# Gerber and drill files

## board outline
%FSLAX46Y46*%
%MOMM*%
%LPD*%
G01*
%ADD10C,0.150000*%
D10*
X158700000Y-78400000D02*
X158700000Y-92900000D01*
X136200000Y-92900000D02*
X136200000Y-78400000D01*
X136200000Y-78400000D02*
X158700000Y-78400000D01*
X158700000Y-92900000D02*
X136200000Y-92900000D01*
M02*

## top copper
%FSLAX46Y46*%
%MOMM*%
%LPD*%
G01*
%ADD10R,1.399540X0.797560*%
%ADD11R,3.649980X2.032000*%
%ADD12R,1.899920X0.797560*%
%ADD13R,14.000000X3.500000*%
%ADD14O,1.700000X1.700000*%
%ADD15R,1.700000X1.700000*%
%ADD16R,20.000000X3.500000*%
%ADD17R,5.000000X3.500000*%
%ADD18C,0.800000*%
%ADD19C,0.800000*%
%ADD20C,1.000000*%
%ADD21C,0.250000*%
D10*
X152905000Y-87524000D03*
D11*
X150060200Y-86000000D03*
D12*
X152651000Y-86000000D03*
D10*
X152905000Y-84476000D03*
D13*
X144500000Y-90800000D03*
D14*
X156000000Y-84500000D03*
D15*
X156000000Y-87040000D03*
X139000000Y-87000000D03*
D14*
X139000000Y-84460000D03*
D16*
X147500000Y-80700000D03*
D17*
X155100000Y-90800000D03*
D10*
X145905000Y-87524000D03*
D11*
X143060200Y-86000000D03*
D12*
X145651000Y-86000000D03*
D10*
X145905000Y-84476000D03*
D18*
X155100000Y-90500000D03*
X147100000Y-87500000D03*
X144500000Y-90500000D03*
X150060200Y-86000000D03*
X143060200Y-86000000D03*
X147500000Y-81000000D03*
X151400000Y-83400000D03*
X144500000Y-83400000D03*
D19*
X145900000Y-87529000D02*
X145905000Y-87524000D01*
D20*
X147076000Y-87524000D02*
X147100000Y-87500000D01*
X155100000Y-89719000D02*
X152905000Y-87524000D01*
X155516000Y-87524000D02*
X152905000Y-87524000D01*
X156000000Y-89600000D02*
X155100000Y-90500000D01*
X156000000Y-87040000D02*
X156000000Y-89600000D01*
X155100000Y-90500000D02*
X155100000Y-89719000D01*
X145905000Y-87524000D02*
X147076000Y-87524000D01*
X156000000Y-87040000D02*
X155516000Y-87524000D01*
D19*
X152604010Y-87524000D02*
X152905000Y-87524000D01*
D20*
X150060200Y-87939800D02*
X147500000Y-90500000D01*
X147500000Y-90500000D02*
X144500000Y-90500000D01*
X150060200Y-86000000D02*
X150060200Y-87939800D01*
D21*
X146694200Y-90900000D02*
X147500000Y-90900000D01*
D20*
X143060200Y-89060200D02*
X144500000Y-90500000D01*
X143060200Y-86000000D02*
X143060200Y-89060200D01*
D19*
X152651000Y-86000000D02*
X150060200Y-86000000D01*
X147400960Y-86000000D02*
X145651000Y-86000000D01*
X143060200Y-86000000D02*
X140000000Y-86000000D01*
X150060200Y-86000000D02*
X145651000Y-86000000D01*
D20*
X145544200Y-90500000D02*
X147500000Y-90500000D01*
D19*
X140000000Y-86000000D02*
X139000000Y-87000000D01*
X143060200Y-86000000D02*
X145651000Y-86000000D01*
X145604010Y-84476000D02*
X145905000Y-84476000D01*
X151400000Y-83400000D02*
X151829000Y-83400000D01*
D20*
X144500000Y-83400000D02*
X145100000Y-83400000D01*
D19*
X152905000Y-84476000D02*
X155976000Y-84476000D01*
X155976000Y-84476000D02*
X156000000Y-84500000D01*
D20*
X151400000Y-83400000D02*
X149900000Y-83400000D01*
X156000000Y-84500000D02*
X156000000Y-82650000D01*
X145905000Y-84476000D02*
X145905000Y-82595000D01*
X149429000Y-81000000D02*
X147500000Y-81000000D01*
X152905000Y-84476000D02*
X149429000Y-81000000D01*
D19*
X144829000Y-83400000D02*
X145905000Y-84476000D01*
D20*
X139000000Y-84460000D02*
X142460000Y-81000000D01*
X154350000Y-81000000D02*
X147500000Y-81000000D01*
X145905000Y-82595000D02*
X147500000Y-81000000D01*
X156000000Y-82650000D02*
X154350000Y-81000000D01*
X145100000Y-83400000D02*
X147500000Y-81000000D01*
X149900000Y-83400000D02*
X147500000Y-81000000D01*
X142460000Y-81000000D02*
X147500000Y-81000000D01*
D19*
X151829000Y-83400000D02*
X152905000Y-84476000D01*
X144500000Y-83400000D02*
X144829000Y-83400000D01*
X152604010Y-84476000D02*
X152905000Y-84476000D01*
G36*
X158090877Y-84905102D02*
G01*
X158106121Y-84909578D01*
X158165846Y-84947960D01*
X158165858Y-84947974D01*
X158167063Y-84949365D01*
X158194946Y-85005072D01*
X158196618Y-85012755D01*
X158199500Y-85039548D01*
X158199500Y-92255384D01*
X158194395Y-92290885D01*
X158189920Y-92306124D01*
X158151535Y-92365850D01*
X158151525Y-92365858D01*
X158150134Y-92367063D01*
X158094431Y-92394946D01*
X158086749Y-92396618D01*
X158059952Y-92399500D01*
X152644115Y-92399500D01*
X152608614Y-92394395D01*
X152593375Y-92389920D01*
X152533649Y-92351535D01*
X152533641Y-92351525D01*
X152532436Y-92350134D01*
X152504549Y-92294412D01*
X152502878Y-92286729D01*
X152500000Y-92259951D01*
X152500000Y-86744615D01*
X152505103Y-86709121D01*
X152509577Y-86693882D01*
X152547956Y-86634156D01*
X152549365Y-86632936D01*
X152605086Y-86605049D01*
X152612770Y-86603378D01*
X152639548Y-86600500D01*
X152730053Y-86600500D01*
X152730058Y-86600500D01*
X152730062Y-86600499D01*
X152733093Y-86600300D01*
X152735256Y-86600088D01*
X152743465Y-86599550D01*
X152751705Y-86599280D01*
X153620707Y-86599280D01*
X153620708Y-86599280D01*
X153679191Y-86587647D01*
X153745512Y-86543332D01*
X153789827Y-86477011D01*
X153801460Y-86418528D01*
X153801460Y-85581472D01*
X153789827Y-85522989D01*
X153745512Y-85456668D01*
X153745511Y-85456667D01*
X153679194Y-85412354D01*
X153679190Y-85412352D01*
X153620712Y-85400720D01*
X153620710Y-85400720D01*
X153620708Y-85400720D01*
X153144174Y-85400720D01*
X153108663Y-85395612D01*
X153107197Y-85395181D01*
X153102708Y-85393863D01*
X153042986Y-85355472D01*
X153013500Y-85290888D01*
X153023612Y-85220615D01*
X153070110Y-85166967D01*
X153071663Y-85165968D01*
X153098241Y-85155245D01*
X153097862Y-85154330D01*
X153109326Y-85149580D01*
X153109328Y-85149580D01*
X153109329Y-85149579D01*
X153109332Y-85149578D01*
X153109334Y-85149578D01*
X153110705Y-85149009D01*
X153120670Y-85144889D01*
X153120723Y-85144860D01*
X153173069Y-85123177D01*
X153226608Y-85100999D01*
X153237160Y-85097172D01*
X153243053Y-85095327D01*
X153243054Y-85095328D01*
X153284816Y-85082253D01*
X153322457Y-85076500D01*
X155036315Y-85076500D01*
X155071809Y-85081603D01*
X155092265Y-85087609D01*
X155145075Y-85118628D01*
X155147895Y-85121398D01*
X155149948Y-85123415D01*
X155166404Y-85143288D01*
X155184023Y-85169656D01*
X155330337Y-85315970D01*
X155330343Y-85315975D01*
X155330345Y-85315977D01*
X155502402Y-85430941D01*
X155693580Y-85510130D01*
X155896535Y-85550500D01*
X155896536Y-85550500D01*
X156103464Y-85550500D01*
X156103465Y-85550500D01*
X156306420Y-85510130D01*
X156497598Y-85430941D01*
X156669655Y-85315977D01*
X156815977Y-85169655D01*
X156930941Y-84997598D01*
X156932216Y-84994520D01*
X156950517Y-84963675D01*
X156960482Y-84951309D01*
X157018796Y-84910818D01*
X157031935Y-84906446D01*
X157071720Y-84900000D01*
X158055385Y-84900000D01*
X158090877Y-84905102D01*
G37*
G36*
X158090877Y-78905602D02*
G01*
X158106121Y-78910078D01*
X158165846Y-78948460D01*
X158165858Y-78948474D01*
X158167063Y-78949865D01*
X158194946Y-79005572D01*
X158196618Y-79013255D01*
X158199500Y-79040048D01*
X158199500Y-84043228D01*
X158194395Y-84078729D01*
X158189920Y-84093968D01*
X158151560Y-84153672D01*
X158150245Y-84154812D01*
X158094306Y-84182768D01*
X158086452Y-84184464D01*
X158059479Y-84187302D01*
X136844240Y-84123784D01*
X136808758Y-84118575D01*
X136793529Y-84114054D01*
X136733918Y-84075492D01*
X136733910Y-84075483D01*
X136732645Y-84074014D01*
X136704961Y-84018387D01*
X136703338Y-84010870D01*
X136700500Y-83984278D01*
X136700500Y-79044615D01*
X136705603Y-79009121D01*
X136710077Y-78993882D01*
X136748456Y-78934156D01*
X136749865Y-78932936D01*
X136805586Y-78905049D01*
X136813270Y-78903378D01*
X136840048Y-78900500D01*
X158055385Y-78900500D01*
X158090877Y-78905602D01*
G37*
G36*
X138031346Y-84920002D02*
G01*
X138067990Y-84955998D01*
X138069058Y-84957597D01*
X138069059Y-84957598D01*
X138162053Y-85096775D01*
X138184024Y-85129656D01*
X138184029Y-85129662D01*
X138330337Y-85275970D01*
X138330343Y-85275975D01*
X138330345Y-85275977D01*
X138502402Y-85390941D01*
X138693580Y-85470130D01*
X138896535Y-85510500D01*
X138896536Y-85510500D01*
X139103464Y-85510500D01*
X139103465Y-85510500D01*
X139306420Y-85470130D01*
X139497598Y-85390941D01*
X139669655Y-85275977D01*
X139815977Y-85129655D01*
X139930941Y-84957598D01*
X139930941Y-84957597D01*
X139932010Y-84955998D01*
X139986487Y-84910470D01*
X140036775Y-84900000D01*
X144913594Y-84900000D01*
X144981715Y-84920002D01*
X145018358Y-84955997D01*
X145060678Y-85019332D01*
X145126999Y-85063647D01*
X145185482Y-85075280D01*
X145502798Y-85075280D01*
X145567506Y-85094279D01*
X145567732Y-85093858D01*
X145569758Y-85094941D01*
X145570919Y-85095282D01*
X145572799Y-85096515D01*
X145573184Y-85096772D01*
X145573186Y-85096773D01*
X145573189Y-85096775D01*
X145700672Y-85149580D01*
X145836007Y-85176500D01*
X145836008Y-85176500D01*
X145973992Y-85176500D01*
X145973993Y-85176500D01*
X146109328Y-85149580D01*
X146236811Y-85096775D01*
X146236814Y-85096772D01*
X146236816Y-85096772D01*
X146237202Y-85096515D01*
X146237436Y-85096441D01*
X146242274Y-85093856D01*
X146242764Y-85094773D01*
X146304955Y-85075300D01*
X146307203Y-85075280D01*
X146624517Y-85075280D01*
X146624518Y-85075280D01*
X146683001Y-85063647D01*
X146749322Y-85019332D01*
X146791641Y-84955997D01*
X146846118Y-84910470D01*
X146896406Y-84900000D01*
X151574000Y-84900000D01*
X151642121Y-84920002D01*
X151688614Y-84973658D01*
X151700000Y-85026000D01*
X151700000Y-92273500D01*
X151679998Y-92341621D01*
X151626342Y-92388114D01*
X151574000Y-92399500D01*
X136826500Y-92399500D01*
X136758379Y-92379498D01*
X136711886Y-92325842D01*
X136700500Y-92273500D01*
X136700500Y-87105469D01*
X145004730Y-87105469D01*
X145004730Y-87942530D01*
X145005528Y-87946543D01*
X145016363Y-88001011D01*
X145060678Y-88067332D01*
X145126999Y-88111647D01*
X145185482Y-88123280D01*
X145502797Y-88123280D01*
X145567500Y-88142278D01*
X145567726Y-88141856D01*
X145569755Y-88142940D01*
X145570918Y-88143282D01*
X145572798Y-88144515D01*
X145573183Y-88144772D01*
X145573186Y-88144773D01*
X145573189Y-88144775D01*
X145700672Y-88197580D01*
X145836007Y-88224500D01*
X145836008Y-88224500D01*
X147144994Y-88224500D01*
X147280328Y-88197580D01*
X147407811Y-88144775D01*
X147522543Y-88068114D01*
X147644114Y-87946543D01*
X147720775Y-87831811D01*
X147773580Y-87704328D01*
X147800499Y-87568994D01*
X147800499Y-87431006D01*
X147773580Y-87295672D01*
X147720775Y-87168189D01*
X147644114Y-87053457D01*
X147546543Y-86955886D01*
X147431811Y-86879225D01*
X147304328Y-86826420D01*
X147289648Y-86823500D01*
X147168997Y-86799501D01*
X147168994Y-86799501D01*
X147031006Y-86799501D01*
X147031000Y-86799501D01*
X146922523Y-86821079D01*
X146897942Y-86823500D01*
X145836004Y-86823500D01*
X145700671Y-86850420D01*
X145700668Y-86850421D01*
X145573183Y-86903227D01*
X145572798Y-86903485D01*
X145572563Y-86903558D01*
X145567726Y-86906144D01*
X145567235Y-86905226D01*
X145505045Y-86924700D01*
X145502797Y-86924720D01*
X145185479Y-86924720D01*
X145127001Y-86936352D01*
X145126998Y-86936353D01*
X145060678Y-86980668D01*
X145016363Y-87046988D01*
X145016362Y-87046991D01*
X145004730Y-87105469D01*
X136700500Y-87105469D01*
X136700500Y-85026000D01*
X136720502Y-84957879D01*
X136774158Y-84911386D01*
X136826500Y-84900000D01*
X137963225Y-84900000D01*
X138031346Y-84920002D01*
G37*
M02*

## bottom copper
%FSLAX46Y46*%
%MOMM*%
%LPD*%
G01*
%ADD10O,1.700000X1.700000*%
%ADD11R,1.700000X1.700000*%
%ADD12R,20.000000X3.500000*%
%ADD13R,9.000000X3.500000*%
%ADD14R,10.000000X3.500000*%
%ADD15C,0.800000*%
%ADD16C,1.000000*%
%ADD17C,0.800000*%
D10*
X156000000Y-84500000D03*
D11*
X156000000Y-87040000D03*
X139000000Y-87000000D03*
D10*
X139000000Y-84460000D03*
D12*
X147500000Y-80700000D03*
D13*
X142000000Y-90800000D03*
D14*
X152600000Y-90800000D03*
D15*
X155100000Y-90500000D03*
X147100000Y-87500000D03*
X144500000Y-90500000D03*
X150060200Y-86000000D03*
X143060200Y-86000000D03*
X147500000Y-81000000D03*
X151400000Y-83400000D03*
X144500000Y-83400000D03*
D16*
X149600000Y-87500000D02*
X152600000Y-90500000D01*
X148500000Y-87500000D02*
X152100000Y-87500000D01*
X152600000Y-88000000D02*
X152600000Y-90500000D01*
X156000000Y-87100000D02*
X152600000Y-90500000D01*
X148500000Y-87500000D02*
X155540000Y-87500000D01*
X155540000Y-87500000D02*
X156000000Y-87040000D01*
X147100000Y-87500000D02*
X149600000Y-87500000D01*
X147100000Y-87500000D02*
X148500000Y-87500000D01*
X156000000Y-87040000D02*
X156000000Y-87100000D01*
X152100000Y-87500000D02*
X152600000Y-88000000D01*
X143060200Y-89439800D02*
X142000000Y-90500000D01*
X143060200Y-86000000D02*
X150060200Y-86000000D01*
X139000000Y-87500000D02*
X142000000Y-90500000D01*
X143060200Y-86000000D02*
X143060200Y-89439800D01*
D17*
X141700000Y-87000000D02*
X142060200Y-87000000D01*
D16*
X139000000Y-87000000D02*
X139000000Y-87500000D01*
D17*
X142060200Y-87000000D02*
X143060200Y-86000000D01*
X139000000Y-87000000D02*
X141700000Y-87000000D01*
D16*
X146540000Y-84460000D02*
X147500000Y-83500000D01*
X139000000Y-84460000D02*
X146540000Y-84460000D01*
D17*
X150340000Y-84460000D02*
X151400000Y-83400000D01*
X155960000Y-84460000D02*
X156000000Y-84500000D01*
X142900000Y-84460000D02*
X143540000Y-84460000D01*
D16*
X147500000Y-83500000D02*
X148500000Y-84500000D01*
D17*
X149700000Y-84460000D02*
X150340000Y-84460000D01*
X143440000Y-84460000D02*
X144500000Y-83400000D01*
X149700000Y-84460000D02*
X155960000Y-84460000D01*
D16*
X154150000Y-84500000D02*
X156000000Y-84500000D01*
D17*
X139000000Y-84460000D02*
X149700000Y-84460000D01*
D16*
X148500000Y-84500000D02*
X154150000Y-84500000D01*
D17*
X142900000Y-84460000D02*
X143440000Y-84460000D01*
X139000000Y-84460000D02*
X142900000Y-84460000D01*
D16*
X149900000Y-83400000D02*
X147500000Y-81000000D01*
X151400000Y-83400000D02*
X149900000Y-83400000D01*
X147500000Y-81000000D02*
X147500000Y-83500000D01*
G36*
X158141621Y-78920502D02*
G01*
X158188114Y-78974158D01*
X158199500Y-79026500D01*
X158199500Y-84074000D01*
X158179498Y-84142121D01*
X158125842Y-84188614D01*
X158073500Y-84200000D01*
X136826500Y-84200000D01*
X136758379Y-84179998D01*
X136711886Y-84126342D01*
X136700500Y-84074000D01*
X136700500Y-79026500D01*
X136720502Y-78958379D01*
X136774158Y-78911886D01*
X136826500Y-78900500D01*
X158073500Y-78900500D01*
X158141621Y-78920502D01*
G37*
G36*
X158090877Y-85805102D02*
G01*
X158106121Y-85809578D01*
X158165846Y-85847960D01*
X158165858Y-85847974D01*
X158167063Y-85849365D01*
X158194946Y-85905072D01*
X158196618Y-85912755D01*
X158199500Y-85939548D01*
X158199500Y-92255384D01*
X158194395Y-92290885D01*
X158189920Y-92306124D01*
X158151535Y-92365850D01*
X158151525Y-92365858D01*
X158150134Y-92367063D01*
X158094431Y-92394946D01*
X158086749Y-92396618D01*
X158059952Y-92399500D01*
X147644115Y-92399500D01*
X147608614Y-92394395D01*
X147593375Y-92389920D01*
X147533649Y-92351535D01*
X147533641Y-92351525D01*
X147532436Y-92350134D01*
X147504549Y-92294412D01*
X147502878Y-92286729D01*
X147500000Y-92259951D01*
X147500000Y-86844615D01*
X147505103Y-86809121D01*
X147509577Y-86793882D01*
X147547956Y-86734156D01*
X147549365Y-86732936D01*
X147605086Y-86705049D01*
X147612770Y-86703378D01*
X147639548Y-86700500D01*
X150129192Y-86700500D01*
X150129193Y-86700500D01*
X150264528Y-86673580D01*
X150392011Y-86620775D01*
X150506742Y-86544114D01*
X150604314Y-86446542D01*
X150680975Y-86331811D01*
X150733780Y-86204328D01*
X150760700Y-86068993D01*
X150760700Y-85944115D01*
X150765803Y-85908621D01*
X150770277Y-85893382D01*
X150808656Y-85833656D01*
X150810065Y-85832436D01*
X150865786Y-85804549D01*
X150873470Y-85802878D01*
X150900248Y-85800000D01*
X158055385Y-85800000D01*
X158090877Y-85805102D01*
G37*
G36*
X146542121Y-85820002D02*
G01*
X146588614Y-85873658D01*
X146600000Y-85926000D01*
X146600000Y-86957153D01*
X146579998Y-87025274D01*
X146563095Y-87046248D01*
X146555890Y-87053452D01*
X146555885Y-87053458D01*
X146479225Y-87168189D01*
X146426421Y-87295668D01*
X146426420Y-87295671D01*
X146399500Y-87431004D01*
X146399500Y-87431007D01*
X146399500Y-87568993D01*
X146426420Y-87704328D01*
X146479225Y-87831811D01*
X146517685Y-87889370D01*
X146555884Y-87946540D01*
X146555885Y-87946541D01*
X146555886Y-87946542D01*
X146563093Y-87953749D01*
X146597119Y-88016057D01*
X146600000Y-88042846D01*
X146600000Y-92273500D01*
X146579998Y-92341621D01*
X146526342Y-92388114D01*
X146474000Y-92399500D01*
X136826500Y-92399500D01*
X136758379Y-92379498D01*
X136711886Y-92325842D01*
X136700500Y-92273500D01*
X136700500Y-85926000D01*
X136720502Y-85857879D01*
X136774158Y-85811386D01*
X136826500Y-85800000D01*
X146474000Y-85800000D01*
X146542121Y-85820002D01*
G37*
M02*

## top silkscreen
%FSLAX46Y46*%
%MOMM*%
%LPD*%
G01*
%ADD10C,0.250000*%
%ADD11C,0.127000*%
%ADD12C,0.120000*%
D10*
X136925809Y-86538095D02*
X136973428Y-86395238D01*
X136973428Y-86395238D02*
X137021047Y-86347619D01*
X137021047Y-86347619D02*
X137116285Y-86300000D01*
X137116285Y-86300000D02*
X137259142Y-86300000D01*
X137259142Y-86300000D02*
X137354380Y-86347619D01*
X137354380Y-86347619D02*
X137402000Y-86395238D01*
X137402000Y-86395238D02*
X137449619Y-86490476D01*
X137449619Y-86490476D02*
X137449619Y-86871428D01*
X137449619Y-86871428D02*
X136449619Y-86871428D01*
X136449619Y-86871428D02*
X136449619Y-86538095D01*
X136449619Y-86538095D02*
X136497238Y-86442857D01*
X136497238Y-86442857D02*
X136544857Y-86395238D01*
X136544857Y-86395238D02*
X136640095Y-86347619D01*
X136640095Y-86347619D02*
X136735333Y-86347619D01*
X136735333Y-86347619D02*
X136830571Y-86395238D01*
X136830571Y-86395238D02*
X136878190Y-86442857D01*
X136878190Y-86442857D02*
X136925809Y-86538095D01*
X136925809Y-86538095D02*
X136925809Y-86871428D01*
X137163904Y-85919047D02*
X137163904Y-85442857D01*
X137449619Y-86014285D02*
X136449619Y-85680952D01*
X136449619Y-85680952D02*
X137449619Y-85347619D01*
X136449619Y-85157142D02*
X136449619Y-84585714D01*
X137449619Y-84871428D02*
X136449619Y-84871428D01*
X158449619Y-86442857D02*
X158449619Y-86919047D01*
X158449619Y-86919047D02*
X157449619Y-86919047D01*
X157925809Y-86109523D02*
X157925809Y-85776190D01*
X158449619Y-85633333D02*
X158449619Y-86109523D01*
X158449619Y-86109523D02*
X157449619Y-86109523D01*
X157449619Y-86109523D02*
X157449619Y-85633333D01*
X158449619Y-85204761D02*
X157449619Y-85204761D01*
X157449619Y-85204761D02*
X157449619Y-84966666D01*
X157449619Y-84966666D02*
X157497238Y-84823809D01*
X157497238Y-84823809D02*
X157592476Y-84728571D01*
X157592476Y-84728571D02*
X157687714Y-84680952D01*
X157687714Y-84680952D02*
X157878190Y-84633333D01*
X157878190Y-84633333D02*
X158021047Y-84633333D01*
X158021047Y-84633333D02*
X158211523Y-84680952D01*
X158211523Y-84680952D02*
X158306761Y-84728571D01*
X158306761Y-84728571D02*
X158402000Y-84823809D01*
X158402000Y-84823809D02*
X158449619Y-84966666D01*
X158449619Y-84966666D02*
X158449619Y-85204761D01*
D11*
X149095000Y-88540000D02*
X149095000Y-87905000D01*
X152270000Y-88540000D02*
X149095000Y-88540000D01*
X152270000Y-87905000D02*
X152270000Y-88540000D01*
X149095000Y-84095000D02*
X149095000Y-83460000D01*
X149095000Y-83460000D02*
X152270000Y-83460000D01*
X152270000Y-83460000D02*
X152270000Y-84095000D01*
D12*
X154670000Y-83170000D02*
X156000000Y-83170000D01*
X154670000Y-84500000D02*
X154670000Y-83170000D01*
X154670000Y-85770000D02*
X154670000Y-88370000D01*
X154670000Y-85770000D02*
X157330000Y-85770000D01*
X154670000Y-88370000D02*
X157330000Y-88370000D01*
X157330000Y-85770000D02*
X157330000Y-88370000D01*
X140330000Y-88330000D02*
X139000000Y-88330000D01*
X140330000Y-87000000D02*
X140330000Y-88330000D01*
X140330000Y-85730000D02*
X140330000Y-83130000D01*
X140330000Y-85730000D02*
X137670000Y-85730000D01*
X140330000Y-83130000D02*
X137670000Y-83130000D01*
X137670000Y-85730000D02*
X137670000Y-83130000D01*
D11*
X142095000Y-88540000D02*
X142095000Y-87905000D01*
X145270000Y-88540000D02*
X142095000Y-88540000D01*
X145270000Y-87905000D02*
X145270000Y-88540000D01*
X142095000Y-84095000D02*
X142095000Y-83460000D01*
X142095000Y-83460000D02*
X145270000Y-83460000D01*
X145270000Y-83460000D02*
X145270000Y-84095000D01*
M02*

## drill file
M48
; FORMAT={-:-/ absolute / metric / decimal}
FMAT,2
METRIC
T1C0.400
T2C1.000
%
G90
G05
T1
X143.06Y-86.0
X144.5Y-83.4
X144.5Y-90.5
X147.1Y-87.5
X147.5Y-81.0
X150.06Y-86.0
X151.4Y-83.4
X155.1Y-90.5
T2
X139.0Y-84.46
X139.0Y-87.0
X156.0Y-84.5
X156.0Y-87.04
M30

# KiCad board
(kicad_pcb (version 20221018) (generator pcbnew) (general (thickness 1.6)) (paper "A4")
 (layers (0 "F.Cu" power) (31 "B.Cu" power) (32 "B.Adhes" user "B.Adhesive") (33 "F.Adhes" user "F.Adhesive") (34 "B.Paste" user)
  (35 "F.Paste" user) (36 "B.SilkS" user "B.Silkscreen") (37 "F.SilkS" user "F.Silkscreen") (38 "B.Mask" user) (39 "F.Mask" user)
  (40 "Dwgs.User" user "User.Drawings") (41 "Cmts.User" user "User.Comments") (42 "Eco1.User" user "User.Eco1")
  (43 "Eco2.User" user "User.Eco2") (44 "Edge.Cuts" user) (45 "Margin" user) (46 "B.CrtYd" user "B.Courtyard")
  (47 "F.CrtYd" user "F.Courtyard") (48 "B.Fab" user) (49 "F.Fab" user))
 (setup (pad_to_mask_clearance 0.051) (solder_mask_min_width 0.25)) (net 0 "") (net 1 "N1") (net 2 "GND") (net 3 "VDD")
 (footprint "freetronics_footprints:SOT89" (layer "F.Cu") (at 151 86 90)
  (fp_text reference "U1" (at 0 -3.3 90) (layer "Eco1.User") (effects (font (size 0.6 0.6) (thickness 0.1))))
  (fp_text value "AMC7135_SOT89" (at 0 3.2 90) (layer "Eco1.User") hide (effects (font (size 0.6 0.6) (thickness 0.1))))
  (fp_line (start -2.54 -1.905) (end -1.905 -1.905) (stroke (width 0.127) (type solid)) (layer "F.SilkS"))
  (fp_line (start -2.54 1.27) (end -2.54 -1.905) (stroke (width 0.127) (type solid)) (layer "F.SilkS"))
  (fp_line (start -1.905 1.27) (end -2.54 1.27) (stroke (width 0.127) (type solid)) (layer "F.SilkS"))
  (fp_line (start 1.905 -1.905) (end 2.54 -1.905) (stroke (width 0.127) (type solid)) (layer "F.SilkS"))
  (fp_line (start 2.54 -1.905) (end 2.54 1.27) (stroke (width 0.127) (type solid)) (layer "F.SilkS"))
  (fp_line (start 2.54 1.27) (end 1.905 1.27) (stroke (width 0.127) (type solid)) (layer "F.SilkS"))
  (pad "1" smd rect (at -1.524 1.905 90) (size 0.79756 1.39954) (layers "F.Cu" "F.Paste" "F.Mask") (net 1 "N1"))
  (pad "2" smd rect (at 0 -0.9398 90) (size 2.032 3.64998) (layers "F.Cu" "F.Paste" "F.Mask") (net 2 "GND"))
  (pad "2" smd rect (at 0 1.651 90) (size 0.79756 1.89992) (layers "F.Cu" "F.Paste" "F.Mask") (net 2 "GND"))
  (pad "3" smd rect (at 1.524 1.905 90) (size 0.79756 1.39954) (layers "F.Cu" "F.Paste" "F.Mask") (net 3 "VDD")))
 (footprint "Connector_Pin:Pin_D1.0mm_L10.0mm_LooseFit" (layer "F.Cu") (at 144.5 90.8)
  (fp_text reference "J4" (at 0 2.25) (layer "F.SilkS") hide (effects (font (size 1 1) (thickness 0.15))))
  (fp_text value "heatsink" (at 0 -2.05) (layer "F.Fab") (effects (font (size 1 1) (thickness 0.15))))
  (pad "1" smd rect (at 0 0) (size 14 3.5) (layers "F.Cu" "F.Paste" "F.Mask") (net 2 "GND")))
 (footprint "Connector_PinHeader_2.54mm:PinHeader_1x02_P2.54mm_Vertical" (layer "F.Cu") (at 156 84.5)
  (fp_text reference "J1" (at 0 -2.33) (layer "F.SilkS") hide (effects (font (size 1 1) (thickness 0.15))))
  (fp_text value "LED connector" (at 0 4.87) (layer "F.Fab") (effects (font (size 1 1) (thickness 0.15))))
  (fp_line (start -1.33 -1.33) (end 0 -1.33) (stroke (width 0.12) (type solid)) (layer "F.SilkS"))
  (fp_line (start -1.33 0) (end -1.33 -1.33) (stroke (width 0.12) (type solid)) (layer "F.SilkS"))
  (fp_line (start -1.33 1.27) (end -1.33 3.87) (stroke (width 0.12) (type solid)) (layer "F.SilkS"))
  (fp_line (start -1.33 1.27) (end 1.33 1.27) (stroke (width 0.12) (type solid)) (layer "F.SilkS"))
  (fp_line (start -1.33 3.87) (end 1.33 3.87) (stroke (width 0.12) (type solid)) (layer "F.SilkS"))
  (fp_line (start 1.33 1.27) (end 1.33 3.87) (stroke (width 0.12) (type solid)) (layer "F.SilkS"))
  (pad "1" thru_hole oval (at 0 0) (size 1.7 1.7) (drill 1) (layers "*.Cu" "*.Mask") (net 3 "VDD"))
  (pad "2" thru_hole rect (at 0 2.54) (size 1.7 1.7) (drill 1) (layers "*.Cu" "*.Mask") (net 1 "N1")))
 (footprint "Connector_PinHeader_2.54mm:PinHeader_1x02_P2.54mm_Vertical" (layer "F.Cu") (at 139 87 180)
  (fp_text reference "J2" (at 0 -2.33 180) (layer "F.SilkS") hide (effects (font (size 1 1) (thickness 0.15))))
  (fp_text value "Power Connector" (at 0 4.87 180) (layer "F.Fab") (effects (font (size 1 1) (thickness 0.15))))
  (fp_line (start -1.33 -1.33) (end 0 -1.33) (stroke (width 0.12) (type solid)) (layer "F.SilkS"))
  (fp_line (start -1.33 0) (end -1.33 -1.33) (stroke (width 0.12) (type solid)) (layer "F.SilkS"))
  (fp_line (start -1.33 1.27) (end -1.33 3.87) (stroke (width 0.12) (type solid)) (layer "F.SilkS"))
  (fp_line (start -1.33 1.27) (end 1.33 1.27) (stroke (width 0.12) (type solid)) (layer "F.SilkS"))
  (fp_line (start -1.33 3.87) (end 1.33 3.87) (stroke (width 0.12) (type solid)) (layer "F.SilkS"))
  (fp_line (start 1.33 1.27) (end 1.33 3.87) (stroke (width 0.12) (type solid)) (layer "F.SilkS"))
  (pad "1" thru_hole rect (at 0 0 180) (size 1.7 1.7) (drill 1) (layers "*.Cu" "*.Mask") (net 2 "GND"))
  (pad "2" thru_hole oval (at 0 2.54 180) (size 1.7 1.7) (drill 1) (layers "*.Cu" "*.Mask") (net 3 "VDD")))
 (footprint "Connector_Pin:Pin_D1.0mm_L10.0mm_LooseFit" (layer "F.Cu") (at 147.5 80.7)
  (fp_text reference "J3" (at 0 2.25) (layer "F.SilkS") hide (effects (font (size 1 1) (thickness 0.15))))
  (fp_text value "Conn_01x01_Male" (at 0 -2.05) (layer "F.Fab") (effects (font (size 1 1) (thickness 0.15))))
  (pad "1" smd rect (at 0 0) (size 20 3.5) (layers "F.Cu" "F.Paste" "F.Mask") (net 3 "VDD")))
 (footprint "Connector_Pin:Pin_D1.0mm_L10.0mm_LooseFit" (layer "F.Cu") (at 155.1 90.8)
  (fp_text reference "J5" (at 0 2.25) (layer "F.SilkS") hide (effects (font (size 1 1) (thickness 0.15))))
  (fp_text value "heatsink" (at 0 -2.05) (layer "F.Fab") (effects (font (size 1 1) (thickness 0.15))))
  (pad "1" smd rect (at 0 0) (size 5 3.5) (layers "F.Cu" "F.Paste" "F.Mask") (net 1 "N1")))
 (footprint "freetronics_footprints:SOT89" (layer "F.Cu") (at 144 86 90)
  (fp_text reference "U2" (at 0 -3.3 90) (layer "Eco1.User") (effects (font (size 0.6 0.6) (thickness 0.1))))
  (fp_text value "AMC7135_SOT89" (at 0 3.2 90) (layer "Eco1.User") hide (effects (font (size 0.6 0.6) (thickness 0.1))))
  (fp_line (start -2.54 -1.905) (end -1.905 -1.905) (stroke (width 0.127) (type solid)) (layer "F.SilkS"))
  (fp_line (start -2.54 1.27) (end -2.54 -1.905) (stroke (width 0.127) (type solid)) (layer "F.SilkS"))
  (fp_line (start -1.905 1.27) (end -2.54 1.27) (stroke (width 0.127) (type solid)) (layer "F.SilkS"))
  (fp_line (start 1.905 -1.905) (end 2.54 -1.905) (stroke (width 0.127) (type solid)) (layer "F.SilkS"))
  (fp_line (start 2.54 -1.905) (end 2.54 1.27) (stroke (width 0.127) (type solid)) (layer "F.SilkS"))
  (fp_line (start 2.54 1.27) (end 1.905 1.27) (stroke (width 0.127) (type solid)) (layer "F.SilkS"))
  (pad "1" smd rect (at -1.524 1.905 90) (size 0.79756 1.39954) (layers "F.Cu" "F.Paste" "F.Mask") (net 1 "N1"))
  (pad "2" smd rect (at 0 -0.9398 90) (size 2.032 3.64998) (layers "F.Cu" "F.Paste" "F.Mask") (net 2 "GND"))
  (pad "2" smd rect (at 0 1.651 90) (size 0.79756 1.89992) (layers "F.Cu" "F.Paste" "F.Mask") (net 2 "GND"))
  (pad "3" smd rect (at 1.524 1.905 90) (size 0.79756 1.39954) (layers "F.Cu" "F.Paste" "F.Mask") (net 3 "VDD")))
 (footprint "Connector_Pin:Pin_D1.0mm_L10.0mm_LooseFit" (layer "B.Cu") (at 147.5 80.7)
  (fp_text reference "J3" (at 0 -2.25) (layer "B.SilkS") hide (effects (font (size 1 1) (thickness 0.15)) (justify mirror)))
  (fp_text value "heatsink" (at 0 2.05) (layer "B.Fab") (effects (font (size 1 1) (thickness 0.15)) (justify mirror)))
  (pad "1" smd rect (at 0 0) (size 20 3.5) (layers "B.Cu" "B.Paste" "B.Mask") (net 3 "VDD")))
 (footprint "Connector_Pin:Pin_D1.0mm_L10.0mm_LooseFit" (layer "B.Cu") (at 142 90.8)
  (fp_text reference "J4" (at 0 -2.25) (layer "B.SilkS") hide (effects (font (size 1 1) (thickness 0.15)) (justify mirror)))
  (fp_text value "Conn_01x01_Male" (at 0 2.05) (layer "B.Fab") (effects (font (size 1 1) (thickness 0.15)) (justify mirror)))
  (pad "1" smd rect (at 0 0) (size 9 3.5) (layers "B.Cu" "B.Paste" "B.Mask") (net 2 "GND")))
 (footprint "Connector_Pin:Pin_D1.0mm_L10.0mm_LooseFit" (layer "B.Cu") (at 152.6 90.8)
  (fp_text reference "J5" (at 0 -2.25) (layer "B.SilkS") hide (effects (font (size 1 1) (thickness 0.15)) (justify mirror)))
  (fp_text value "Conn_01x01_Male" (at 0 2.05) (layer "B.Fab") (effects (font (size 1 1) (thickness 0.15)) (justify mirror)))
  (pad "1" smd rect (at 0 0) (size 10 3.5) (layers "B.Cu" "B.Paste" "B.Mask") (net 1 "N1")))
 (gr_line (start 158.7 78.4) (end 158.7 92.9) (stroke (width 0.15) (type solid)) (layer "Edge.Cuts"))
 (gr_line (start 136.2 92.9) (end 136.2 78.4) (stroke (width 0.15) (type solid)) (layer "Edge.Cuts"))
 (gr_line (start 136.2 78.4) (end 158.7 78.4) (stroke (width 0.15) (type solid)) (layer "Edge.Cuts"))
 (gr_line (start 158.7 92.9) (end 136.2 92.9) (stroke (width 0.15) (type solid)) (layer "Edge.Cuts"))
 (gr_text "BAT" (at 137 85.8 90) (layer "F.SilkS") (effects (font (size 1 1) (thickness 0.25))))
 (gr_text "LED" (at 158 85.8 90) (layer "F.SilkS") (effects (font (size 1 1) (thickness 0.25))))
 (segment (start 145.9 87.529) (end 145.905 87.524) (width 0.8) (layer "F.Cu") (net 1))
 (segment (start 147.076 87.524) (end 147.1 87.5) (width 1) (layer "F.Cu") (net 1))
 (segment (start 155.1 89.719) (end 152.905 87.524) (width 1) (layer "F.Cu") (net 1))
 (segment (start 155.516 87.524) (end 152.905 87.524) (width 1) (layer "F.Cu") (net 1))
 (segment (start 156 89.6) (end 155.1 90.5) (width 1) (layer "F.Cu") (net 1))
 (segment (start 156 87.04) (end 156 89.6) (width 1) (layer "F.Cu") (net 1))
 (segment (start 155.1 90.5) (end 155.1 89.719) (width 1) (layer "F.Cu") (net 1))
 (segment (start 145.905 87.524) (end 147.076 87.524) (width 1) (layer "F.Cu") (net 1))
 (segment (start 156 87.04) (end 155.516 87.524) (width 1) (layer "F.Cu") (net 1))
 (segment (start 152.60401 87.524) (end 152.905 87.524) (width 0.8) (layer "F.Cu") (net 1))
 (via (at 155.1 90.5) (size 0.8) (drill 0.4) (layers "F.Cu" "B.Cu") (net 1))
 (via (at 147.1 87.5) (size 0.8) (drill 0.4) (layers "F.Cu" "B.Cu") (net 1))
 (segment (start 149.6 87.5) (end 152.6 90.5) (width 1) (layer "B.Cu") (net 1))
 (segment (start 148.5 87.5) (end 152.1 87.5) (width 1) (layer "B.Cu") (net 1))
 (segment (start 152.6 88) (end 152.6 90.5) (width 1) (layer "B.Cu") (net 1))
 (segment (start 156 87.1) (end 152.6 90.5) (width 1) (layer "B.Cu") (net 1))
 (segment (start 148.5 87.5) (end 155.54 87.5) (width 1) (layer "B.Cu") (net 1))
 (segment (start 155.54 87.5) (end 156 87.04) (width 1) (layer "B.Cu") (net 1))
 (segment (start 147.1 87.5) (end 149.6 87.5) (width 1) (layer "B.Cu") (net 1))
 (segment (start 147.1 87.5) (end 148.5 87.5) (width 1) (layer "B.Cu") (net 1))
 (segment (start 156 87.04) (end 156 87.1) (width 1) (layer "B.Cu") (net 1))
 (segment (start 152.1 87.5) (end 152.6 88) (width 1) (layer "B.Cu") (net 1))
 (segment (start 150.0602 87.9398) (end 147.5 90.5) (width 1) (layer "F.Cu") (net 2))
 (segment (start 147.5 90.5) (end 144.5 90.5) (width 1) (layer "F.Cu") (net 2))
 (segment (start 150.0602 86) (end 150.0602 87.9398) (width 1) (layer "F.Cu") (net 2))
 (segment (start 146.6942 90.9) (end 147.5 90.9) (width 0.25) (layer "F.Cu") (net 2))
 (segment (start 143.0602 89.0602) (end 144.5 90.5) (width 1) (layer "F.Cu") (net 2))
 (segment (start 143.0602 86) (end 143.0602 89.0602) (width 1) (layer "F.Cu") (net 2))
 (segment (start 152.651 86) (end 150.0602 86) (width 0.8) (layer "F.Cu") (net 2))
 (segment (start 147.40096 86) (end 145.651 86) (width 0.8) (layer "F.Cu") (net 2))
 (segment (start 143.0602 86) (end 140 86) (width 0.8) (layer "F.Cu") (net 2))
 (segment (start 150.0602 86) (end 145.651 86) (width 0.8) (layer "F.Cu") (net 2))
 (segment (start 145.5442 90.5) (end 147.5 90.5) (width 1) (layer "F.Cu") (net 2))
 (segment (start 140 86) (end 139 87) (width 0.8) (layer "F.Cu") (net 2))
 (segment (start 143.0602 86) (end 145.651 86) (width 0.8) (layer "F.Cu") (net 2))
 (via (at 144.5 90.5) (size 0.8) (drill 0.4) (layers "F.Cu" "B.Cu") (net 2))
 (via (at 150.0602 86) (size 0.8) (drill 0.4) (layers "F.Cu" "B.Cu") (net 2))
 (via (at 143.0602 86) (size 0.8) (drill 0.4) (layers "F.Cu" "B.Cu") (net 2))
 (segment (start 143.0602 89.4398) (end 142 90.5) (width 1) (layer "B.Cu") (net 2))
 (segment (start 143.0602 86) (end 150.0602 86) (width 1) (layer "B.Cu") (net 2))
 (segment (start 139 87.5) (end 142 90.5) (width 1) (layer "B.Cu") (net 2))
 (segment (start 143.0602 86) (end 143.0602 89.4398) (width 1) (layer "B.Cu") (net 2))
 (segment (start 141.7 87) (end 142.0602 87) (width 0.8) (layer "B.Cu") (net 2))
 (segment (start 139 87) (end 139 87.5) (width 1) (layer "B.Cu") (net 2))
 (segment (start 142.0602 87) (end 143.0602 86) (width 0.8) (layer "B.Cu") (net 2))
 (segment (start 139 87) (end 141.7 87) (width 0.8) (layer "B.Cu") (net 2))
 (segment (start 145.60401 84.476) (end 145.905 84.476) (width 0.8) (layer "F.Cu") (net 3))
 (segment (start 151.4 83.4) (end 151.829 83.4) (width 0.8) (layer "F.Cu") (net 3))
 (segment (start 144.5 83.4) (end 145.1 83.4) (width 1) (layer "F.Cu") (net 3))
 (segment (start 152.905 84.476) (end 155.976 84.476) (width 0.8) (layer "F.Cu") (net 3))
 (segment (start 155.976 84.476) (end 156 84.5) (width 0.8) (layer "F.Cu") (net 3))
 (segment (start 151.4 83.4) (end 149.9 83.4) (width 1) (layer "F.Cu") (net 3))
 (segment (start 156 84.5) (end 156 82.65) (width 1) (layer "F.Cu") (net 3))
 (segment (start 145.905 84.476) (end 145.905 82.595) (width 1) (layer "F.Cu") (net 3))
 (segment (start 149.429 81) (end 147.5 81) (width 1) (layer "F.Cu") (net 3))
 (segment (start 152.905 84.476) (end 149.429 81) (width 1) (layer "F.Cu") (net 3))
 (segment (start 144.829 83.4) (end 145.905 84.476) (width 0.8) (layer "F.Cu") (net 3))
 (segment (start 139 84.46) (end 142.46 81) (width 1) (layer "F.Cu") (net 3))
 (segment (start 154.35 81) (end 147.5 81) (width 1) (layer "F.Cu") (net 3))
 (segment (start 145.905 82.595) (end 147.5 81) (width 1) (layer "F.Cu") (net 3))
 (segment (start 156 82.65) (end 154.35 81) (width 1) (layer "F.Cu") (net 3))
 (segment (start 145.1 83.4) (end 147.5 81) (width 1) (layer "F.Cu") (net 3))
 (segment (start 149.9 83.4) (end 147.5 81) (width 1) (layer "F.Cu") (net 3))
 (segment (start 142.46 81) (end 147.5 81) (width 1) (layer "F.Cu") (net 3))
 (segment (start 151.829 83.4) (end 152.905 84.476) (width 0.8) (layer "F.Cu") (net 3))
 (segment (start 144.5 83.4) (end 144.829 83.4) (width 0.8) (layer "F.Cu") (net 3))
 (segment (start 152.60401 84.476) (end 152.905 84.476) (width 0.8) (layer "F.Cu") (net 3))
 (via (at 147.5 81) (size 0.8) (drill 0.4) (layers "F.Cu" "B.Cu") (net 3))
 (via (at 151.4 83.4) (size 0.8) (drill 0.4) (layers "F.Cu" "B.Cu") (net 3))
 (via (at 144.5 83.4) (size 0.8) (drill 0.4) (layers "F.Cu" "B.Cu") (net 3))
 (segment (start 146.54 84.46) (end 147.5 83.5) (width 1) (layer "B.Cu") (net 3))
 (segment (start 139 84.46) (end 146.54 84.46) (width 1) (layer "B.Cu") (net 3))
 (segment (start 150.34 84.46) (end 151.4 83.4) (width 0.8) (layer "B.Cu") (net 3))
 (segment (start 155.96 84.46) (end 156 84.5) (width 0.8) (layer "B.Cu") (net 3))
 (segment (start 142.9 84.46) (end 143.54 84.46) (width 0.8) (layer "B.Cu") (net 3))
 (segment (start 147.5 83.5) (end 148.5 84.5) (width 1) (layer "B.Cu") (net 3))
 (segment (start 149.7 84.46) (end 150.34 84.46) (width 0.8) (layer "B.Cu") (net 3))
 (segment (start 143.44 84.46) (end 144.5 83.4) (width 0.8) (layer "B.Cu") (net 3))
 (segment (start 149.7 84.46) (end 155.96 84.46) (width 0.8) (layer "B.Cu") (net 3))
 (segment (start 154.15 84.5) (end 156 84.5) (width 1) (layer "B.Cu") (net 3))
 (segment (start 139 84.46) (end 149.7 84.46) (width 0.8) (layer "B.Cu") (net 3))
 (segment (start 148.5 84.5) (end 154.15 84.5) (width 1) (layer "B.Cu") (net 3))
 (segment (start 142.9 84.46) (end 143.44 84.46) (width 0.8) (layer "B.Cu") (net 3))
 (segment (start 139 84.46) (end 142.9 84.46) (width 0.8) (layer "B.Cu") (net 3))
 (segment (start 149.9 83.4) (end 147.5 81) (width 1) (layer "B.Cu") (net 3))
 (segment (start 151.4 83.4) (end 149.9 83.4) (width 1) (layer "B.Cu") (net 3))
 (segment (start 147.5 81) (end 147.5 83.5) (width 1) (layer "B.Cu") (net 3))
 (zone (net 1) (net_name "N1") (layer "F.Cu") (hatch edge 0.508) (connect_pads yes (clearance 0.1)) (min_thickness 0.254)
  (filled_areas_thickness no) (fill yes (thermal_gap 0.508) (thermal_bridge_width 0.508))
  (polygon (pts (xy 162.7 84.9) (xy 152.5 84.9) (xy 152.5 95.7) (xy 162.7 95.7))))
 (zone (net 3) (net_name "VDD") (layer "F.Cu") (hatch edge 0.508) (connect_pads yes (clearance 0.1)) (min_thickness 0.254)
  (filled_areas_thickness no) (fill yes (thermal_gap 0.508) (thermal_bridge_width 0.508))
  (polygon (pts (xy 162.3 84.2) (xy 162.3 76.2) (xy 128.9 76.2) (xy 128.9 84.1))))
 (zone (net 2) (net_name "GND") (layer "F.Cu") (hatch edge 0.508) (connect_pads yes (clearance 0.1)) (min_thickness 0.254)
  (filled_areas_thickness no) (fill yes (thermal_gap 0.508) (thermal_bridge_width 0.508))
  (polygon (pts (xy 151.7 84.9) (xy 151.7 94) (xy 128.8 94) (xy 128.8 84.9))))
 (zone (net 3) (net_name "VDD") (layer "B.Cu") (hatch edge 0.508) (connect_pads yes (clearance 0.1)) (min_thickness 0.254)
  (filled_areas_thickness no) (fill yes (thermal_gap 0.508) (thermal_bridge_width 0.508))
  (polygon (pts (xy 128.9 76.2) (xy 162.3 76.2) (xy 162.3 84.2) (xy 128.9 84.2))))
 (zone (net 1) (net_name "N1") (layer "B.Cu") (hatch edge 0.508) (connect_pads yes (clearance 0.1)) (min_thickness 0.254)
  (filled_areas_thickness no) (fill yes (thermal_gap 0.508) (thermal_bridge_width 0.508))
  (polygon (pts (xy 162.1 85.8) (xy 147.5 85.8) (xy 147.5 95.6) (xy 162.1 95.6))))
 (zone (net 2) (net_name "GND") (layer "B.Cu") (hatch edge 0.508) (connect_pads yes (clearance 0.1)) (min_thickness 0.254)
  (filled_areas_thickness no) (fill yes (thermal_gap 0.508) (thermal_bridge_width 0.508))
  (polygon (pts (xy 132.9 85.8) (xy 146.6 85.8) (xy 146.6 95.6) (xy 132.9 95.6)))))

